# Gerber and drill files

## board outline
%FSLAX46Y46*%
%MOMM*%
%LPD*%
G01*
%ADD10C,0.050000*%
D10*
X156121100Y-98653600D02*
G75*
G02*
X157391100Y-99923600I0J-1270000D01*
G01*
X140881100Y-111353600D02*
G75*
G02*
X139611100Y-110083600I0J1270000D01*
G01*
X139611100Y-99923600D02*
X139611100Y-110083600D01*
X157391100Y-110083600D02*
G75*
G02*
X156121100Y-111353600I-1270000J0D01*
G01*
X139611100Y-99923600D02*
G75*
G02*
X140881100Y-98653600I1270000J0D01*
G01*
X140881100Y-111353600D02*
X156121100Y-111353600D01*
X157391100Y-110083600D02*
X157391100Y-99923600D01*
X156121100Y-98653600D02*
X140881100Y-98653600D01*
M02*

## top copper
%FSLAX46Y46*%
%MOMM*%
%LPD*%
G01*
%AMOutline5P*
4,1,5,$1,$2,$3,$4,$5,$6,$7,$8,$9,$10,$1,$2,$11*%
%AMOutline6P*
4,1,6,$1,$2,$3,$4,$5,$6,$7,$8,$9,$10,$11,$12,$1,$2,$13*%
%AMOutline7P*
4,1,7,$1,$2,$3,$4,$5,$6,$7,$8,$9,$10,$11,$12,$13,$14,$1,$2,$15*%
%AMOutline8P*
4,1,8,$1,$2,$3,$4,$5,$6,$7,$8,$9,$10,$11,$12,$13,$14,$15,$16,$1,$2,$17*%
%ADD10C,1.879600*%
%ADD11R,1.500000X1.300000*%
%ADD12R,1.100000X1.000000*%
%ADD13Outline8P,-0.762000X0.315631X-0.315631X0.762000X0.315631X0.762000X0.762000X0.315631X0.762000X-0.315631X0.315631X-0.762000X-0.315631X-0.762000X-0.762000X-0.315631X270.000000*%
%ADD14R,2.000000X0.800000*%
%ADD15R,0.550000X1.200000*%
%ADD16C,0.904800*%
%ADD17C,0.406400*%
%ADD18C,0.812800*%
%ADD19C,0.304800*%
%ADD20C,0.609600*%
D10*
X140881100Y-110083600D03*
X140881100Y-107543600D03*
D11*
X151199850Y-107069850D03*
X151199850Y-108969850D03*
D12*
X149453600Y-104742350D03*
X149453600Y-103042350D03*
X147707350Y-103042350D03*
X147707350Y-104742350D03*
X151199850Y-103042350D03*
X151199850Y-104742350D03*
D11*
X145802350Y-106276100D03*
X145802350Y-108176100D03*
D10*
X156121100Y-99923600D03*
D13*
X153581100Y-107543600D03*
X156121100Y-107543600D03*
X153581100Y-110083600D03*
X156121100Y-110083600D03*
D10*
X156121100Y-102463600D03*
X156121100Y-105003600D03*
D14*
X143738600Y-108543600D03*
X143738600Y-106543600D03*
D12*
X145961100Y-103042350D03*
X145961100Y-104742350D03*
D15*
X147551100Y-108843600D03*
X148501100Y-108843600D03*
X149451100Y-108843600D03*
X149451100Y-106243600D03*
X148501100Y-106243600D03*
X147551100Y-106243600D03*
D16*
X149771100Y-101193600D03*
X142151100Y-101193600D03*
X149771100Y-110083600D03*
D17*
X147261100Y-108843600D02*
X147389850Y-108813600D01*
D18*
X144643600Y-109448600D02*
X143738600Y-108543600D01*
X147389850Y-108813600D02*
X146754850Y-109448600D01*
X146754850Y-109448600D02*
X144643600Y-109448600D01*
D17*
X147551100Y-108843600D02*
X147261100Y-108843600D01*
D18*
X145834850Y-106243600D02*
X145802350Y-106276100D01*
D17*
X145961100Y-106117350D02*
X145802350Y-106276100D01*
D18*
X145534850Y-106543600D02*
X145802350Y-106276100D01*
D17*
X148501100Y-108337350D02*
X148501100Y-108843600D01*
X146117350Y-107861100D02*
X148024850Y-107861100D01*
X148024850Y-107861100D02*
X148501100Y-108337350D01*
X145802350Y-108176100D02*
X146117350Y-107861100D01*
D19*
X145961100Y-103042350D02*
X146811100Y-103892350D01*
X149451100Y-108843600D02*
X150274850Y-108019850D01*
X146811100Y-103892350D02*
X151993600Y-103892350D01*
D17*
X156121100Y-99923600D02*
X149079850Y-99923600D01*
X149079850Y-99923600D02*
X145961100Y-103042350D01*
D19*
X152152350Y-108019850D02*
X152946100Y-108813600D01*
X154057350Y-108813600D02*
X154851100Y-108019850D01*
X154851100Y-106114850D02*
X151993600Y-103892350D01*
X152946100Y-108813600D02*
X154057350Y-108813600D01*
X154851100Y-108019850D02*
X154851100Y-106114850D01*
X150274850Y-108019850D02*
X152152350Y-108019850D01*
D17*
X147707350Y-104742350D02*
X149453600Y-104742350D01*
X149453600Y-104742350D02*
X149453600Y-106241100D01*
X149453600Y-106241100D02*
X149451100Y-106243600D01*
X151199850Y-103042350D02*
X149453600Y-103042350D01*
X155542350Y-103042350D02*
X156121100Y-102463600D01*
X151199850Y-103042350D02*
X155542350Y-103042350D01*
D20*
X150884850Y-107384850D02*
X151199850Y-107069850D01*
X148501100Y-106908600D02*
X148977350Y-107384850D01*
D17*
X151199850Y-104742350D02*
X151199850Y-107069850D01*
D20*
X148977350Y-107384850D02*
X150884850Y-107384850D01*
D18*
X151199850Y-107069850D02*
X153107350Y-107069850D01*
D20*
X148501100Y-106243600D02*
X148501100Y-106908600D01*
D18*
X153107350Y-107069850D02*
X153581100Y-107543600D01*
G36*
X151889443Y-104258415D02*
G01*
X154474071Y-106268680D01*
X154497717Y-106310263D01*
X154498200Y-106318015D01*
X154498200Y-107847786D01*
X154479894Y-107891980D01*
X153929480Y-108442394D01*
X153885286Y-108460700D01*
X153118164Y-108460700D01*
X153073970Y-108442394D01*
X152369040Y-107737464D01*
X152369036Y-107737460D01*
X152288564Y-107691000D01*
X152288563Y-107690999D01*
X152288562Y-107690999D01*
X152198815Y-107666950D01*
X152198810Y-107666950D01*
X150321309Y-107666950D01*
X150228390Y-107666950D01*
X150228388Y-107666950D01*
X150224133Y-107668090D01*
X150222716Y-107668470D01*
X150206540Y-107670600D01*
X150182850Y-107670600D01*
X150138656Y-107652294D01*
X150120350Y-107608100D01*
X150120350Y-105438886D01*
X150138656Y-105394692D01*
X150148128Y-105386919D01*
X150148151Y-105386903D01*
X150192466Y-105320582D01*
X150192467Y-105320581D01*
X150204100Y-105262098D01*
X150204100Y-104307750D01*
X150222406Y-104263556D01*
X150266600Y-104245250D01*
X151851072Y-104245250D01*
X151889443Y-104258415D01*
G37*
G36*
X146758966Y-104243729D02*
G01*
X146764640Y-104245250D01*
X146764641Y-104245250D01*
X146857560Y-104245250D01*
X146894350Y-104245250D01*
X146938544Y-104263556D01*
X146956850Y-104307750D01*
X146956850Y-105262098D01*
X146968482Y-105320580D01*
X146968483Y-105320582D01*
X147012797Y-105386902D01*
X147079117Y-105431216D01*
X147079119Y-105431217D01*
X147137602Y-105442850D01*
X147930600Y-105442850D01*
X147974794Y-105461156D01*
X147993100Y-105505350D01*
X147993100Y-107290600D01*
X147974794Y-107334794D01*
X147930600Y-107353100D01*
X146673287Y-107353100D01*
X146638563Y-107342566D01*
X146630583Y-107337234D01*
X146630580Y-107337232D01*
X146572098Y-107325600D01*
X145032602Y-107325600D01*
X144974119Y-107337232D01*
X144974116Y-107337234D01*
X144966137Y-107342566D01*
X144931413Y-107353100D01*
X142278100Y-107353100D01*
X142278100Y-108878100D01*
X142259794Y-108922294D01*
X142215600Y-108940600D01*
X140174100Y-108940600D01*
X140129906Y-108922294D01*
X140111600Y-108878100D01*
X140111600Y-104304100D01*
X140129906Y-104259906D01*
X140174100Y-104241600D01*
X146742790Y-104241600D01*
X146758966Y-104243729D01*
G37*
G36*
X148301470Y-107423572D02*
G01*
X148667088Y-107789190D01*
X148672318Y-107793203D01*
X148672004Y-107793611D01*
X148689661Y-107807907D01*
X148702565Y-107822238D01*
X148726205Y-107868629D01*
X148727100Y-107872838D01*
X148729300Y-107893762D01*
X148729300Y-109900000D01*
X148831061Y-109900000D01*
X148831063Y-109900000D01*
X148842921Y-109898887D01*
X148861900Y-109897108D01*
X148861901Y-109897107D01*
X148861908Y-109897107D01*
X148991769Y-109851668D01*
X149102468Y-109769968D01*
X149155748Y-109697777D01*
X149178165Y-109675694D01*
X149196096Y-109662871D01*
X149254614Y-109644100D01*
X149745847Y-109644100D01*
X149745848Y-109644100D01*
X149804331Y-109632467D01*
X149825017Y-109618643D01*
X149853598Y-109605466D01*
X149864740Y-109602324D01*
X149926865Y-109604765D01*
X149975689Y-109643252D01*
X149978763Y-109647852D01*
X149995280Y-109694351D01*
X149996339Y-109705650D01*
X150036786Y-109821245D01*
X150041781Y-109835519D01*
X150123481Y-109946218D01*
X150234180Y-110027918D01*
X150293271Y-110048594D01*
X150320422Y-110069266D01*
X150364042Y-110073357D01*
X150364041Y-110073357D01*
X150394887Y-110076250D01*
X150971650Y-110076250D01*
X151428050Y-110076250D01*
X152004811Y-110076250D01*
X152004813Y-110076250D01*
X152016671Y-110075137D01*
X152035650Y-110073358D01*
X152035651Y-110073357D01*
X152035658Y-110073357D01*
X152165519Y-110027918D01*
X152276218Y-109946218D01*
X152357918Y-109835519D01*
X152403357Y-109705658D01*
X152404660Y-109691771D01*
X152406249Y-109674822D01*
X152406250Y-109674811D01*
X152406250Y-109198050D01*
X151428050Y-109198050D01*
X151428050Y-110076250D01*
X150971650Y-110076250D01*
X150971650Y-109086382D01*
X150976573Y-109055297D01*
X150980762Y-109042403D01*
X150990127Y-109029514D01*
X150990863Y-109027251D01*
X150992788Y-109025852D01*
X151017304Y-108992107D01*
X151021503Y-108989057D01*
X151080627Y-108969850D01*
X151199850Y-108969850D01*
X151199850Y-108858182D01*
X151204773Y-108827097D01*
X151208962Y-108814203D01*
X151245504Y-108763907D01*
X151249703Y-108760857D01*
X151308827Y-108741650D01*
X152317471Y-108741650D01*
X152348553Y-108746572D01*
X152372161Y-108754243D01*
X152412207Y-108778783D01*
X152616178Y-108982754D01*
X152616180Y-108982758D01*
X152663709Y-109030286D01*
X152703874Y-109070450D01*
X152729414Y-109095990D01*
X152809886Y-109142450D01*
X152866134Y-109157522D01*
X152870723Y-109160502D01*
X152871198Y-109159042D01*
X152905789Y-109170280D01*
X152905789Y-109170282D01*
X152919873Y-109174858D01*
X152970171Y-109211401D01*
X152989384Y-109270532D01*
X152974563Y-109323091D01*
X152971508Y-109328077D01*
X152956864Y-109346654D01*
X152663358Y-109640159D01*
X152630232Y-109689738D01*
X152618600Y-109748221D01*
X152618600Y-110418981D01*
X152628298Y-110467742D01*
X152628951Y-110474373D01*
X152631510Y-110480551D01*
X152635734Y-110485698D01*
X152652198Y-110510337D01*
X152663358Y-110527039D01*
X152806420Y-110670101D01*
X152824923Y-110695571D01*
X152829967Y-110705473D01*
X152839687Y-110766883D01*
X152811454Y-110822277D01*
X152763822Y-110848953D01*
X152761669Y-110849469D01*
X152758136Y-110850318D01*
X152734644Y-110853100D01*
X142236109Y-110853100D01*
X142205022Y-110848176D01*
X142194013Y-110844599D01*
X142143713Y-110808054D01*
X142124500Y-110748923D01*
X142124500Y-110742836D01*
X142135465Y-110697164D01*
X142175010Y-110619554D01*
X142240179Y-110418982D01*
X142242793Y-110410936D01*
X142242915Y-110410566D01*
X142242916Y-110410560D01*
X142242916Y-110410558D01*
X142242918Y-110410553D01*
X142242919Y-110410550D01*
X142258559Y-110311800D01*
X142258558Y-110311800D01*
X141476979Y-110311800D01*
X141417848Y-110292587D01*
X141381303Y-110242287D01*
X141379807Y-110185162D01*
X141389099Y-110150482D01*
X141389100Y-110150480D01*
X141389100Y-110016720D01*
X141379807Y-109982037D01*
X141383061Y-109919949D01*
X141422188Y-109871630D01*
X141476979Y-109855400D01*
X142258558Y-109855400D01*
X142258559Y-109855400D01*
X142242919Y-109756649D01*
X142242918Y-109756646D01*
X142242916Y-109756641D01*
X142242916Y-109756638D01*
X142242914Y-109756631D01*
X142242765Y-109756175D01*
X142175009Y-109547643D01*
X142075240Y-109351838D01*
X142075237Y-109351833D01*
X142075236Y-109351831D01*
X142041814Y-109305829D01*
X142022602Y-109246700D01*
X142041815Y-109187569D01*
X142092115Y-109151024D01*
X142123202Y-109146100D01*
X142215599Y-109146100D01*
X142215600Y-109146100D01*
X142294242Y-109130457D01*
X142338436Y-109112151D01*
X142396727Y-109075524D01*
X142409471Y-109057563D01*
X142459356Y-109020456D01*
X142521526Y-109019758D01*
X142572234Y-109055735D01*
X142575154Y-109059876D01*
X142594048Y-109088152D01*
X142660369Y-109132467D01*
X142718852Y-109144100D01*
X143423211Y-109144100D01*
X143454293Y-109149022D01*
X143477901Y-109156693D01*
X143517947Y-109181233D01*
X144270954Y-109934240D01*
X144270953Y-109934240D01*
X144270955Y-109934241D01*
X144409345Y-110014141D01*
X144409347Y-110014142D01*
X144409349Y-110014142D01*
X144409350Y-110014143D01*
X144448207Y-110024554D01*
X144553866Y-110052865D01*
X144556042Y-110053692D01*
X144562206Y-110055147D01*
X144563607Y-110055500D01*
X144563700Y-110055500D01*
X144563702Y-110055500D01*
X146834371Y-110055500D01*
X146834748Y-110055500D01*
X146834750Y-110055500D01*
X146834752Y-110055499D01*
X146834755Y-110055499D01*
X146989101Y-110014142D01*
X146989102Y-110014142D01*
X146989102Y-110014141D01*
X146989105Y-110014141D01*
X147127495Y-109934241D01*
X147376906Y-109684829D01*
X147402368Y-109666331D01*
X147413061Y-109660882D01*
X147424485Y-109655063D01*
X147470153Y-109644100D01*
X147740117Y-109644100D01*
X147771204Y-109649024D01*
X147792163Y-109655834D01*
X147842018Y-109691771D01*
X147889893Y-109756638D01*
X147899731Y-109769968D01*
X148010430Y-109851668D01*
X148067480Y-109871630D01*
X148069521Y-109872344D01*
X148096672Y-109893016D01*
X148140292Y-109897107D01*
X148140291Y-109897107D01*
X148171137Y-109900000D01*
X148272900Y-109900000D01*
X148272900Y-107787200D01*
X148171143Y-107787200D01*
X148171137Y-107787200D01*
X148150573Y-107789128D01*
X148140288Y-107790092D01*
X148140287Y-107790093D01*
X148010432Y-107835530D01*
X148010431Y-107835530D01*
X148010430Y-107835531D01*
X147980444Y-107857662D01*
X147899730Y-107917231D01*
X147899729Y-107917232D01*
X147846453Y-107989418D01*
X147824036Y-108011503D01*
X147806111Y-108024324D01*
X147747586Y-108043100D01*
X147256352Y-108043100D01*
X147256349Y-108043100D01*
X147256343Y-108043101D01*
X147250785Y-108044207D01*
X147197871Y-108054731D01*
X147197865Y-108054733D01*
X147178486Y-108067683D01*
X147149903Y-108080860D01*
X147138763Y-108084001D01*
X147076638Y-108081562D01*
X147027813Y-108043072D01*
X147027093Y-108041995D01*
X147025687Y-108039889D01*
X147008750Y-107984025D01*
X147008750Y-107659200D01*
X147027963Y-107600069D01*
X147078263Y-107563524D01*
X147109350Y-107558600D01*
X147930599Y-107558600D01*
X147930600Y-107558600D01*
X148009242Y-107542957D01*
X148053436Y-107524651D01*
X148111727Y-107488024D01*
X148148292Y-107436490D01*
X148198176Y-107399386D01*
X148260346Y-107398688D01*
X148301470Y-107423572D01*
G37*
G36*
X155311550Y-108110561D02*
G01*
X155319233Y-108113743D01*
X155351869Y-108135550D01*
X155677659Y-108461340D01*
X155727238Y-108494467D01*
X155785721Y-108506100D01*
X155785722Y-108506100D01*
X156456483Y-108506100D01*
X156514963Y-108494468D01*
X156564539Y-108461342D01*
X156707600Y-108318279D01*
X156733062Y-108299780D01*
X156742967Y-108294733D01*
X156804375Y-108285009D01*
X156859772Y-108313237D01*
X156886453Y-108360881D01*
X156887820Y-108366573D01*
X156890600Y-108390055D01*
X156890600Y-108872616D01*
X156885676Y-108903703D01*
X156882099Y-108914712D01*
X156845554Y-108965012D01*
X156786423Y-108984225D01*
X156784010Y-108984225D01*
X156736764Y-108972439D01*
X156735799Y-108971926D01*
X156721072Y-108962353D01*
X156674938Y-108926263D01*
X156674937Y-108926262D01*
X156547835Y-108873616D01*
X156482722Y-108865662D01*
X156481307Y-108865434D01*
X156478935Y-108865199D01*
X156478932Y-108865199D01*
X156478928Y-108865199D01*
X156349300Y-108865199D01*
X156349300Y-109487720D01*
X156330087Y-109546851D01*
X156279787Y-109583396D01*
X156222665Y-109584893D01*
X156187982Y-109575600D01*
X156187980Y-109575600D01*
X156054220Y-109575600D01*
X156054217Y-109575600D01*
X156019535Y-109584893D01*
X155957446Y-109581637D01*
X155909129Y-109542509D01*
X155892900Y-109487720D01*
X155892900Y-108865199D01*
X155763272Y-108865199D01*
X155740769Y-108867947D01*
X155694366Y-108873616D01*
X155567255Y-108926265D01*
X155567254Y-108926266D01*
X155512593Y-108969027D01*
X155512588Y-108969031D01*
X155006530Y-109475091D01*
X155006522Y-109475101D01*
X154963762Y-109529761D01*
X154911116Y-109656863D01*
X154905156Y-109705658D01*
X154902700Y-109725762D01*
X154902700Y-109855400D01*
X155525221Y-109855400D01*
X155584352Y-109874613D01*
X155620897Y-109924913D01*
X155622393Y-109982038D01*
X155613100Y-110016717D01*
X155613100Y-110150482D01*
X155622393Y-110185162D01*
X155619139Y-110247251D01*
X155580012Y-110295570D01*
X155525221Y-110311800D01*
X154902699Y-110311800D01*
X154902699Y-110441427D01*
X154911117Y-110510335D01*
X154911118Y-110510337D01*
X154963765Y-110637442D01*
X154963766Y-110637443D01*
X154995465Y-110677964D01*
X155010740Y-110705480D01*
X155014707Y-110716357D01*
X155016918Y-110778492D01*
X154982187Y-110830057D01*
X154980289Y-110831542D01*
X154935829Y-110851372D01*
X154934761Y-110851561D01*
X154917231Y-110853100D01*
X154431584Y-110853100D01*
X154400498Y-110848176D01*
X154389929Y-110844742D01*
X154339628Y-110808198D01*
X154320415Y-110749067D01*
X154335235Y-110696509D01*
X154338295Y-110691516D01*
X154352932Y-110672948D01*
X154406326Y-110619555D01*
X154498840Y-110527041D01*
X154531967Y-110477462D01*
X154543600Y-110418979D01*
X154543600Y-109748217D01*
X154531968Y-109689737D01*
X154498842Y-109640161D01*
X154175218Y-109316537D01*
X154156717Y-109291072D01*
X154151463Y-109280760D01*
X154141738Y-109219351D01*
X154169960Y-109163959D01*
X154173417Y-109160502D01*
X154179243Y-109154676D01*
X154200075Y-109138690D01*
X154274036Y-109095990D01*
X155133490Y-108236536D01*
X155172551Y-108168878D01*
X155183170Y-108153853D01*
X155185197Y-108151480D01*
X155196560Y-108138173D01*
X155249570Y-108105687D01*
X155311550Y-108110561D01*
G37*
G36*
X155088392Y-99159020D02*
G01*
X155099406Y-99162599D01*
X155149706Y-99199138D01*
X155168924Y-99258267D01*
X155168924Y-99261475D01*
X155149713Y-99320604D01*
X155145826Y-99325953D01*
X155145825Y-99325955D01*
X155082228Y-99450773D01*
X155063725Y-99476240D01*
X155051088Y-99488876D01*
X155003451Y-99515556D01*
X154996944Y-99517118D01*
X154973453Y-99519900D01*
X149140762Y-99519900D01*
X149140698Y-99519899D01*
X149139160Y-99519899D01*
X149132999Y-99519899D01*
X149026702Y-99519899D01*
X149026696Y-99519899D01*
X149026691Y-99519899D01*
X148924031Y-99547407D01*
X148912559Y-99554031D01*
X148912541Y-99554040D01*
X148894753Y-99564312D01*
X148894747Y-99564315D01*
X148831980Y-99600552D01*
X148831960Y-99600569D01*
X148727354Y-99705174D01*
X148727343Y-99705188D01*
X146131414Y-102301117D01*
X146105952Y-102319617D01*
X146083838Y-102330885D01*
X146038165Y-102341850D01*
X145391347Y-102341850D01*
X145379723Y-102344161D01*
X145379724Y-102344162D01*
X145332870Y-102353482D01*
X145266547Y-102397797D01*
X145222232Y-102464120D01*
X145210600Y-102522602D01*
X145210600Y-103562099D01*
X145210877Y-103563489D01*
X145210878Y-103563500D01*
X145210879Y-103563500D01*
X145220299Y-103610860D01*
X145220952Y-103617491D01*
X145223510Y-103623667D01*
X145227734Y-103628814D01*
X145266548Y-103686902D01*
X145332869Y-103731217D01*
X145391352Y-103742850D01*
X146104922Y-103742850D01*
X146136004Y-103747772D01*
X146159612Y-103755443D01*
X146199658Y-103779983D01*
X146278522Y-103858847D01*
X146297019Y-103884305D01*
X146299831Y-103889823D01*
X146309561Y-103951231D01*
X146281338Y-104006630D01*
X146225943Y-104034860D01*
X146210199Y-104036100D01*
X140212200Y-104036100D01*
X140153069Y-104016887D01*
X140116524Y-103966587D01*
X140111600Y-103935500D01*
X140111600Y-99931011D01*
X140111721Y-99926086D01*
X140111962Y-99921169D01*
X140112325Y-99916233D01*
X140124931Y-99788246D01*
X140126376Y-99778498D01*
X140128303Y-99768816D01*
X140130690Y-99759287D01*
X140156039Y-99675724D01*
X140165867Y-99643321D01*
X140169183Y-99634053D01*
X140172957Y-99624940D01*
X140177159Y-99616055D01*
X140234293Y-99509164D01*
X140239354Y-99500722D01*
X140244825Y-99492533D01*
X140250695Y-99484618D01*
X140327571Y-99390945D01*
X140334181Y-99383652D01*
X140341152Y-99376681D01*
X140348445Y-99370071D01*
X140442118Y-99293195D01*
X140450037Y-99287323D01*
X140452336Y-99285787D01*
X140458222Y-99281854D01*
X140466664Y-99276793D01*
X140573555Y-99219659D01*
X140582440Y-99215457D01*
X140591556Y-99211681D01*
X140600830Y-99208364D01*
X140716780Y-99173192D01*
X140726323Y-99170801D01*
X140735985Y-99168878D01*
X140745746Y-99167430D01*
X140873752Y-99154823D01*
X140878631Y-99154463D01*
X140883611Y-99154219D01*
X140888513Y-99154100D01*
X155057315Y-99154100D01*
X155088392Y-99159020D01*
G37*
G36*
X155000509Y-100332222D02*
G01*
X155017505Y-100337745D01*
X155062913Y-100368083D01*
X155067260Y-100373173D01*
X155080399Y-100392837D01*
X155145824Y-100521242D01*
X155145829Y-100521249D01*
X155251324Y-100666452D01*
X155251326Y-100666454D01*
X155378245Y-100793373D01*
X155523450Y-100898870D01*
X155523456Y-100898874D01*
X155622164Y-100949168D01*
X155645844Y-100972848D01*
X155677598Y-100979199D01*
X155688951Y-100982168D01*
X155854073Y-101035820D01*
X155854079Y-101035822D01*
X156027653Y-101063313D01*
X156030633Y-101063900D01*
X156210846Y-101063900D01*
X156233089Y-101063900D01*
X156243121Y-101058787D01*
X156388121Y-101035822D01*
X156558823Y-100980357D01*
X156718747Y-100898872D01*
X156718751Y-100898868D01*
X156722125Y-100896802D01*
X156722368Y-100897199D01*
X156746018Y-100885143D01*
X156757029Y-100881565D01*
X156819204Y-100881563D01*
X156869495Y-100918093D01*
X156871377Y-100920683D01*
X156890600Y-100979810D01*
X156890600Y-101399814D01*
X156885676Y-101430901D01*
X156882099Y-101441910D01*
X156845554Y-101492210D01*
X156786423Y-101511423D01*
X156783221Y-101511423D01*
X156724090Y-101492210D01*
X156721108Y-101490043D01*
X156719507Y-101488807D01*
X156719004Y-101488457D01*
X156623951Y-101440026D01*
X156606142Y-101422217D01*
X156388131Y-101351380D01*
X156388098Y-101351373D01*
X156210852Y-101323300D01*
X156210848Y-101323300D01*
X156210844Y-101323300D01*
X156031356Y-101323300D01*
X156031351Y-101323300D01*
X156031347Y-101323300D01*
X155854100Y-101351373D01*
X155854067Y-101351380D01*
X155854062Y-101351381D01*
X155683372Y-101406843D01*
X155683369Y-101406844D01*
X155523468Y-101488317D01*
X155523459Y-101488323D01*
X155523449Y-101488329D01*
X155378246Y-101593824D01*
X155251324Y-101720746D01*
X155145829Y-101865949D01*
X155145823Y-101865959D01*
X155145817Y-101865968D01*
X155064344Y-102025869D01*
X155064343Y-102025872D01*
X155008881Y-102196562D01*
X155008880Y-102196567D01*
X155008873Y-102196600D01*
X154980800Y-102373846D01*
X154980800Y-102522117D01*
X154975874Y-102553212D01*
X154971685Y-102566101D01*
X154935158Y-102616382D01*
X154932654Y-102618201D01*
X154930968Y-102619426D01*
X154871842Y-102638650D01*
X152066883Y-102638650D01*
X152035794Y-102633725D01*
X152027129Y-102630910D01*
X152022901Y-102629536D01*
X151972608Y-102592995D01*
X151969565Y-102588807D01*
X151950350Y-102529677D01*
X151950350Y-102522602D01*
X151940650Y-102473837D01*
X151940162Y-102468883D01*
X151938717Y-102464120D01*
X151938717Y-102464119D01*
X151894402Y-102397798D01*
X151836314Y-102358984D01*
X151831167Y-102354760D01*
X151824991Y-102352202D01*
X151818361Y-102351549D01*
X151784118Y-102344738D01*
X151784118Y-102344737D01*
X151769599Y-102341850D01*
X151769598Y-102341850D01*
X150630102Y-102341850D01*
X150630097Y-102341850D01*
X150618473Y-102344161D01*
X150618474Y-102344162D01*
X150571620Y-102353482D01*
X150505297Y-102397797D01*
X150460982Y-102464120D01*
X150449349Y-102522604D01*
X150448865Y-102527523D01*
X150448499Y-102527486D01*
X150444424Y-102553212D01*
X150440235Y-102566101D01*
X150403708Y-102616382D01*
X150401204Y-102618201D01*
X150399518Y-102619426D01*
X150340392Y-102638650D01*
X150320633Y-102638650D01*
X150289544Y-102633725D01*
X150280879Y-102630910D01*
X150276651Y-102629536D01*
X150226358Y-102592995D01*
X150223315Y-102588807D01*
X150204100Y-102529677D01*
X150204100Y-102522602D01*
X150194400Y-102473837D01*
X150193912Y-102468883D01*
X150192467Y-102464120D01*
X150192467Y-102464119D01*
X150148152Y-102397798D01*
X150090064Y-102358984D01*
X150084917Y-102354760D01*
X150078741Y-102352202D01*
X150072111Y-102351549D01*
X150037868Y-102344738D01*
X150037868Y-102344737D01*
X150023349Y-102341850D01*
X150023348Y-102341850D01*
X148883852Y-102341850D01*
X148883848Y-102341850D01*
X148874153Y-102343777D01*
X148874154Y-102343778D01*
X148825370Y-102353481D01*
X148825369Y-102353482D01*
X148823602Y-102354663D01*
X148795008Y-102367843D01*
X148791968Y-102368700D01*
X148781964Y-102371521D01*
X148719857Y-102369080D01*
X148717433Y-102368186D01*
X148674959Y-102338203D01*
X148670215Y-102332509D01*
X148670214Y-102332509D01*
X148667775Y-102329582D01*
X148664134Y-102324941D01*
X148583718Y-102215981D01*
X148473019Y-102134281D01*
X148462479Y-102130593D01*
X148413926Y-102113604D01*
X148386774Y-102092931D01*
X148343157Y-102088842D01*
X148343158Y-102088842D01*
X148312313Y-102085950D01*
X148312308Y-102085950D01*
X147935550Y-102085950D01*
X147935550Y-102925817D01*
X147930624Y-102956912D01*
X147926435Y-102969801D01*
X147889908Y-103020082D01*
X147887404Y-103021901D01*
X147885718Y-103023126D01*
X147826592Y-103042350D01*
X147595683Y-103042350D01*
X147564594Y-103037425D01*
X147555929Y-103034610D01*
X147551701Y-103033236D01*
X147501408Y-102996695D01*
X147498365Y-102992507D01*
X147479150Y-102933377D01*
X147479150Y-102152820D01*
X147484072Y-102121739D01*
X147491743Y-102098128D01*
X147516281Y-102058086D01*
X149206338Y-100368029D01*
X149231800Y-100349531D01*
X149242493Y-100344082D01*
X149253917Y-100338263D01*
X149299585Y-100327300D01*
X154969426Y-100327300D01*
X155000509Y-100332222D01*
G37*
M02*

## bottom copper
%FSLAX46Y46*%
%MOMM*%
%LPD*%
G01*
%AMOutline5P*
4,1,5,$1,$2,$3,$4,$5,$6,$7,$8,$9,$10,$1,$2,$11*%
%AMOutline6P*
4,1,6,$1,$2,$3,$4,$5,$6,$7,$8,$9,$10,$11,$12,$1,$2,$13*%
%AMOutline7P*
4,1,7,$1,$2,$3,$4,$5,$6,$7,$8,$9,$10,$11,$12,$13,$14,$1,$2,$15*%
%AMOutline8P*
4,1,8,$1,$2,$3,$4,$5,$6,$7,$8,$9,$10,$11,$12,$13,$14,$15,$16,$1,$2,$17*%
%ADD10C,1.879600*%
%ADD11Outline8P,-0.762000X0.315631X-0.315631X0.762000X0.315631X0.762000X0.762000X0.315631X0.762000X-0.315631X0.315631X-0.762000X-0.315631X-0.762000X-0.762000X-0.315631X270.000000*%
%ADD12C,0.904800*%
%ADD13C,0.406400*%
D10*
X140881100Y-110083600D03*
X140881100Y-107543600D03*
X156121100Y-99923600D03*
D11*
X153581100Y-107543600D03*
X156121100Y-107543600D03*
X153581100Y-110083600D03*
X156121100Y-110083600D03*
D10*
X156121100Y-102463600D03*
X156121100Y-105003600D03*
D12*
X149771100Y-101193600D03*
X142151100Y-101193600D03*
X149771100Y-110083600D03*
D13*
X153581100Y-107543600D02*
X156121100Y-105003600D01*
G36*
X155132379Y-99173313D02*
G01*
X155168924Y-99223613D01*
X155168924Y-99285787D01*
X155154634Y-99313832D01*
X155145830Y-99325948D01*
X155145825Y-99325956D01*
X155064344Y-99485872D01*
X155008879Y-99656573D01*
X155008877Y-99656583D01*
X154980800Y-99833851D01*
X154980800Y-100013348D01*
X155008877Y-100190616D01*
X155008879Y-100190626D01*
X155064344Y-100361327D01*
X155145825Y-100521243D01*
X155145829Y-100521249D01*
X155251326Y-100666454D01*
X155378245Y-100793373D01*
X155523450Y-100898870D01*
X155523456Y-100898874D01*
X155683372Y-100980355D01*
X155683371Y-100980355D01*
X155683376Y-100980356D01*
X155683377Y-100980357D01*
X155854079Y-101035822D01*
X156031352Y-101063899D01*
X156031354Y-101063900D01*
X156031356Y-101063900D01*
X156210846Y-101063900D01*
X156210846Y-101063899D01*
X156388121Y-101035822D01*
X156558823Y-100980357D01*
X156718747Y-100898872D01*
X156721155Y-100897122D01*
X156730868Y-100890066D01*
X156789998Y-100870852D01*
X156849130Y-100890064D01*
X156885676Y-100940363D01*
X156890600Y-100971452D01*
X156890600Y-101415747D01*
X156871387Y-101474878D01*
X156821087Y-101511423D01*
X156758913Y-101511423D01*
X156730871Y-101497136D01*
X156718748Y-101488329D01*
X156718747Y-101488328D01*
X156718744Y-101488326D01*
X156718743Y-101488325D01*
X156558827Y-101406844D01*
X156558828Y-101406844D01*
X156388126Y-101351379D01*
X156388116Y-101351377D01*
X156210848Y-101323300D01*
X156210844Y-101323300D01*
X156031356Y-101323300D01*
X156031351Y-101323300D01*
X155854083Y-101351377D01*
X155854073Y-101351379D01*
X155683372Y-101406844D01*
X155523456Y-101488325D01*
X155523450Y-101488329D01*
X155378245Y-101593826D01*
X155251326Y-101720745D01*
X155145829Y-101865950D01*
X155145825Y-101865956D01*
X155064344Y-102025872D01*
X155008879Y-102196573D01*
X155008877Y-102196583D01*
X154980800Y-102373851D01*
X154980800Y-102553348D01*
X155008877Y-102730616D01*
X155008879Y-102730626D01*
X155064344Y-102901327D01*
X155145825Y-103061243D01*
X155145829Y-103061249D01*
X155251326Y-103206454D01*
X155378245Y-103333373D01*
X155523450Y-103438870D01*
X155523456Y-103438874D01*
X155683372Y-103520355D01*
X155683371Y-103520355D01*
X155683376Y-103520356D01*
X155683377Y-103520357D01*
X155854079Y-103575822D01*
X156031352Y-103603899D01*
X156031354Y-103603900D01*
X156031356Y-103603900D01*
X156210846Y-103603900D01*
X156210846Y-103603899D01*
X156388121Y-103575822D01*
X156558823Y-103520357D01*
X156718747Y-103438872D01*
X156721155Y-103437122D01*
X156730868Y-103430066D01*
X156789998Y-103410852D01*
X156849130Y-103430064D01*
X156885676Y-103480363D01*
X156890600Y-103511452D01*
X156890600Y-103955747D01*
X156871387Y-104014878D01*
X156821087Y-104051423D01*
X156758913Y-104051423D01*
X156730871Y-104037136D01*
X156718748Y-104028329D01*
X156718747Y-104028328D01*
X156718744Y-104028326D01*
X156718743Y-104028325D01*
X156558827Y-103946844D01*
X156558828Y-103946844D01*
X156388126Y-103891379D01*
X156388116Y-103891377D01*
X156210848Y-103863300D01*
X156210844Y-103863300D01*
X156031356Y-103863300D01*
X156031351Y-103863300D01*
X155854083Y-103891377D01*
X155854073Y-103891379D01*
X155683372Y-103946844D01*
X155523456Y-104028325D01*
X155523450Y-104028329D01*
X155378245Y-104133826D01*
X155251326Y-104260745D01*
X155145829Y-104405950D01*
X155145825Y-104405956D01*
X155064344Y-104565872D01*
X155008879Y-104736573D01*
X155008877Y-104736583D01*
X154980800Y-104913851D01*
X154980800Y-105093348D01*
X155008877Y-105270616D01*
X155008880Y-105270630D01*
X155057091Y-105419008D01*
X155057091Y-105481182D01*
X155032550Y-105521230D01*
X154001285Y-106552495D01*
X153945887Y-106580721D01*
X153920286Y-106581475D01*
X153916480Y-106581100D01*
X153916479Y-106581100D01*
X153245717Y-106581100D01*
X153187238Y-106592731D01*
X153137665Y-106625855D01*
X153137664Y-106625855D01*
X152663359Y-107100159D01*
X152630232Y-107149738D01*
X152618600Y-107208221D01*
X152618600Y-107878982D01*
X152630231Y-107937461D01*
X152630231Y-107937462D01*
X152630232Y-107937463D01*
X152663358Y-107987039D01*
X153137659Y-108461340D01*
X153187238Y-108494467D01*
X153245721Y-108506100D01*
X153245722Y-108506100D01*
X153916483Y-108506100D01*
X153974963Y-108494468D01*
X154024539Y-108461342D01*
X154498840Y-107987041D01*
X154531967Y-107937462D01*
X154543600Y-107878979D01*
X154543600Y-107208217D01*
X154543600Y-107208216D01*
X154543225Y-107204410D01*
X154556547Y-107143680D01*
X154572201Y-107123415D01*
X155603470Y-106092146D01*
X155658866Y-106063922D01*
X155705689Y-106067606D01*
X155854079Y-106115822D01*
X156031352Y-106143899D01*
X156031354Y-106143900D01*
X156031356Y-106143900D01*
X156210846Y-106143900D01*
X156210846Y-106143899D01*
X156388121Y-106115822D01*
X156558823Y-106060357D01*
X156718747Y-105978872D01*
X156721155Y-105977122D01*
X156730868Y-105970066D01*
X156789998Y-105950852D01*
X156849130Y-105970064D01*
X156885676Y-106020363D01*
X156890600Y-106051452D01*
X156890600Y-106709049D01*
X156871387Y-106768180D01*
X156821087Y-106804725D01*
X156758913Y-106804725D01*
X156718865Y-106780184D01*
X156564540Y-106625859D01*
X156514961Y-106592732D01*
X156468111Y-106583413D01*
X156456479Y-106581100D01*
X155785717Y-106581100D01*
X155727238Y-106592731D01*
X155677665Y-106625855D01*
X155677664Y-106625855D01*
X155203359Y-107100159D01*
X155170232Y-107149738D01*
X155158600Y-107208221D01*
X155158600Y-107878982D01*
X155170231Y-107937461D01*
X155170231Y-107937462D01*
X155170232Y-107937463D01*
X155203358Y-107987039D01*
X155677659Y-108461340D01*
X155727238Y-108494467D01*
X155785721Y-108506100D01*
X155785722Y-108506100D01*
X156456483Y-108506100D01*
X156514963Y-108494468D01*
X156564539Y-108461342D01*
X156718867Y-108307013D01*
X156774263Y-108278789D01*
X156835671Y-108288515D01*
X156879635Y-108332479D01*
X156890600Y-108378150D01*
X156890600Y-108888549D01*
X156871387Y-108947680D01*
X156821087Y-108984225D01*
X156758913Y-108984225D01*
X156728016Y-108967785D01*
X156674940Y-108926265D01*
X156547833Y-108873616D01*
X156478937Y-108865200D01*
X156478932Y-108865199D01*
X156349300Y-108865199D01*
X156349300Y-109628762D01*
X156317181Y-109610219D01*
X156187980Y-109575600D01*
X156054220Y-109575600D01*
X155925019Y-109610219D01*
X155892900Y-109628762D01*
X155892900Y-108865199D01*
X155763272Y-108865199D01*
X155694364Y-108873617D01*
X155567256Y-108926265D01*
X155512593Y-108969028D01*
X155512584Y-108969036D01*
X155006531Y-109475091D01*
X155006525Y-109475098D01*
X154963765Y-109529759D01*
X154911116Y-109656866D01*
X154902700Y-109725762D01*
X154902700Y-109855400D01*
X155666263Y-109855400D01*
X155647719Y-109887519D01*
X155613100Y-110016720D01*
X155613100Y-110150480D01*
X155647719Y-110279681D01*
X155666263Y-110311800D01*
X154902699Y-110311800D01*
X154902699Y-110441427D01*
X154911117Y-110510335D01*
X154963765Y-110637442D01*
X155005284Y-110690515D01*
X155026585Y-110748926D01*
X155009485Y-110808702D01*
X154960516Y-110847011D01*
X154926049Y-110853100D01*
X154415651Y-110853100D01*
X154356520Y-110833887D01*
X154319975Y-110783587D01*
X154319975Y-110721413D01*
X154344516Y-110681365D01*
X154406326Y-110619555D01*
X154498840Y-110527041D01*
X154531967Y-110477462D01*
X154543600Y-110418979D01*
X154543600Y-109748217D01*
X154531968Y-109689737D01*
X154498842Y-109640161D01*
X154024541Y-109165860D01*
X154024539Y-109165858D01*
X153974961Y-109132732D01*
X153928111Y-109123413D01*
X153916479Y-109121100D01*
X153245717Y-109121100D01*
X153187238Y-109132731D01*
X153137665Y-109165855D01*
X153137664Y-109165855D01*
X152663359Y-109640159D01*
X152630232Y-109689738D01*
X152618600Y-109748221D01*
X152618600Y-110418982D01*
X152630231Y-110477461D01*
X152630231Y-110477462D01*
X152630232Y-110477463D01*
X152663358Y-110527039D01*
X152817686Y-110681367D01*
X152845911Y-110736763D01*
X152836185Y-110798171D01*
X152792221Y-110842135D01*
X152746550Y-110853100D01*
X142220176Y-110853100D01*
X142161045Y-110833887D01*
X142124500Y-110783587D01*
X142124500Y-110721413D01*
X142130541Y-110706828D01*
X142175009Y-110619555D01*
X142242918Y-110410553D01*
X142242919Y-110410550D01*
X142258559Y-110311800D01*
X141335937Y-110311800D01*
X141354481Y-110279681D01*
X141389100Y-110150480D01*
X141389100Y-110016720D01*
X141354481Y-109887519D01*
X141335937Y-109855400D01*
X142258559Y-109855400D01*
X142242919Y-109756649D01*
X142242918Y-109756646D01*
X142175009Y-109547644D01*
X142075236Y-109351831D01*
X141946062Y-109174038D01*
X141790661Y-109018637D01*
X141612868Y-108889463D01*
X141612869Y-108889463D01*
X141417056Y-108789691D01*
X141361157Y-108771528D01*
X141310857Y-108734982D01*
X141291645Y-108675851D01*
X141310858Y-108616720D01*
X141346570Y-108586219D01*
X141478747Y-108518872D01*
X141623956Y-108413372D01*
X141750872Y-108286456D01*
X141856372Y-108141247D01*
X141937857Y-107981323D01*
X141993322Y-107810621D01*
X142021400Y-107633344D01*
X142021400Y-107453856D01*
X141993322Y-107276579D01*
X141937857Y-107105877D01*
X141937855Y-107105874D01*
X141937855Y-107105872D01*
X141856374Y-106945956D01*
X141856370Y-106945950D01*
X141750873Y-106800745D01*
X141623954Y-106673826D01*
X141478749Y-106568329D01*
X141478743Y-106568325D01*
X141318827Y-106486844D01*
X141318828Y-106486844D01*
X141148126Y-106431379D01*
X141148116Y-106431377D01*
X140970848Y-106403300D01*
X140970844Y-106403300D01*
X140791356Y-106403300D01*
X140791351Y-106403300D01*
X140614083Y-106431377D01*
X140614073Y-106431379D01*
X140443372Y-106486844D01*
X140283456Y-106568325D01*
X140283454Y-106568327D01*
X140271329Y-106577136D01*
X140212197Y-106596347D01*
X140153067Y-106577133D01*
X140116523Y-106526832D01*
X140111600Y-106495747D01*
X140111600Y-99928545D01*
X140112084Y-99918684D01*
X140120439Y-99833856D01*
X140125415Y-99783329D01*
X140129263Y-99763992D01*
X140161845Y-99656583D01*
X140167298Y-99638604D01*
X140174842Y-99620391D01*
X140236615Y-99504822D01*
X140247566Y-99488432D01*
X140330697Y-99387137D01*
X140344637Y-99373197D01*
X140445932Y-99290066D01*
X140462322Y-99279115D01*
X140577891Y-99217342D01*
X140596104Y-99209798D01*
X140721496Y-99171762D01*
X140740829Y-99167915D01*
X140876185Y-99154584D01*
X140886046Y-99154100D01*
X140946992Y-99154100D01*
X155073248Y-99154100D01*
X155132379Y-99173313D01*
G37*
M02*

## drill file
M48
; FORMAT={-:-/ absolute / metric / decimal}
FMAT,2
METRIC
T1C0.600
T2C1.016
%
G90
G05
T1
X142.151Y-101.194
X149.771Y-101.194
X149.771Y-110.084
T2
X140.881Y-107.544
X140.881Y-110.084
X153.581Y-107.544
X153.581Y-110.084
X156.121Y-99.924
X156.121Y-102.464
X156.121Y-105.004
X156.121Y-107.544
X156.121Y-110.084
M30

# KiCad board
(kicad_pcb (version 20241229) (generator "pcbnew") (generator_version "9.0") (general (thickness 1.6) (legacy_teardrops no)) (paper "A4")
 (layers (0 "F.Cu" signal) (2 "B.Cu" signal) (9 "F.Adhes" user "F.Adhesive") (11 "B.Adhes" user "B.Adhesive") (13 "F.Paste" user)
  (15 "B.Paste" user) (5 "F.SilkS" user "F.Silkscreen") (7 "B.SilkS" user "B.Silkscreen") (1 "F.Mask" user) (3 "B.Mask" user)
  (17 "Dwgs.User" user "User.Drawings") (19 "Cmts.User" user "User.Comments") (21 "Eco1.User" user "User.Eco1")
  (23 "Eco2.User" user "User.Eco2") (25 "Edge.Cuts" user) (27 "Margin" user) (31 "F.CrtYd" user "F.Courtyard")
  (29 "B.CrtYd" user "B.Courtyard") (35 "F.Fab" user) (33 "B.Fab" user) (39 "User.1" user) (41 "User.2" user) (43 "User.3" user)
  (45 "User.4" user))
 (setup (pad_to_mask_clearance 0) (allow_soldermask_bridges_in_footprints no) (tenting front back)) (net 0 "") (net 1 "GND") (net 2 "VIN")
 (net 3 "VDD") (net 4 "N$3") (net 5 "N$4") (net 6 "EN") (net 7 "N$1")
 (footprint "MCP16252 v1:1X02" (layer "F.Cu") (at 140.8811 110.0836 90)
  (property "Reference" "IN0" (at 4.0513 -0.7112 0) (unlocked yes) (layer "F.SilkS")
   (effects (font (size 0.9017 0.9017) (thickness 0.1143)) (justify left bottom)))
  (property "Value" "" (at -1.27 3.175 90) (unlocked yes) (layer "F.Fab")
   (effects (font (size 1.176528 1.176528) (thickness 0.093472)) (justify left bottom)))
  (pad "1" thru_hole circle (at 0 0 180) (size 1.8796 1.8796) (drill 1.016) (layers "*.Cu" "*.Mask") (remove_unused_layers no) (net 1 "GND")
   (solder_mask_margin 0.0508) (thermal_bridge_angle 0))
  (pad "2" thru_hole circle (at 2.54 0 180) (size 1.8796 1.8796) (drill 1.016) (layers "*.Cu" "*.Mask") (remove_unused_layers no)
   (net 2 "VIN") (solder_mask_margin 0.0508) (thermal_bridge_angle 0)))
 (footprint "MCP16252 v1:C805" (layer "F.Cu") (at 151.19985 108.01985 -90)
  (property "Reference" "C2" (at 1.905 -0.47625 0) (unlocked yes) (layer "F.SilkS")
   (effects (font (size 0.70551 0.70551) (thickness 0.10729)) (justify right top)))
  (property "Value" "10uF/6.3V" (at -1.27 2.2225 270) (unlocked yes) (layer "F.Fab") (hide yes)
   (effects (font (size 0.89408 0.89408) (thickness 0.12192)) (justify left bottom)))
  (pad "1" smd rect (at -0.95 0 270) (size 1.3 1.5) (layers "F.Cu" "F.Mask" "F.Paste") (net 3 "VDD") (solder_mask_margin 0.0508)
   (solder_paste_margin 0) (thermal_bridge_angle 0))
  (pad "2" smd rect (at 0.95 0 270) (size 1.3 1.5) (layers "F.Cu" "F.Mask" "F.Paste") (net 1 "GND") (solder_mask_margin 0.0508)
   (solder_paste_margin 0) (thermal_bridge_angle 0)))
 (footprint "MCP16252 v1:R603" (layer "F.Cu") (at 149.4536 103.89235 90)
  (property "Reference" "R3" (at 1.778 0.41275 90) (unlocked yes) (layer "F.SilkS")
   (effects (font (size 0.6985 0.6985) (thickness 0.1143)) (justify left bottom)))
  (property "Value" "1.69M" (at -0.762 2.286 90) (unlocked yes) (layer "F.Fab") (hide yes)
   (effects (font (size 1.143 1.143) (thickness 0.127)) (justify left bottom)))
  (pad "1" smd rect (at -0.85 0 90) (size 1 1.1) (layers "F.Cu" "F.Mask" "F.Paste") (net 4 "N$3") (solder_mask_margin 0.0508)
   (solder_paste_margin 0) (thermal_bridge_angle 0))
  (pad "2" smd rect (at 0.85 0 90) (size 1 1.1) (layers "F.Cu" "F.Mask" "F.Paste") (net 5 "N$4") (solder_mask_margin 0.0508)
   (solder_paste_margin 0) (thermal_bridge_angle 0)))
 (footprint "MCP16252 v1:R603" (layer "F.Cu") (at 147.70735 103.89235 -90)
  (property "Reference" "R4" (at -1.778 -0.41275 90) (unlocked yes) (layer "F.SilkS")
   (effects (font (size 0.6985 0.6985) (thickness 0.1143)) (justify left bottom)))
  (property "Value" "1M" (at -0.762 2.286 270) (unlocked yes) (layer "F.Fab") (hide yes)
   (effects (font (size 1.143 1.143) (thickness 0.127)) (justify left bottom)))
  (pad "1" smd rect (at -0.85 0 270) (size 1 1.1) (layers "F.Cu" "F.Mask" "F.Paste") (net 1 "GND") (solder_mask_margin 0.0508)
   (solder_paste_margin 0) (thermal_bridge_angle 0))
  (pad "2" smd rect (at 0.85 0 270) (size 1 1.1) (layers "F.Cu" "F.Mask" "F.Paste") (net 4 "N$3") (solder_mask_margin 0.0508)
   (solder_paste_margin 0) (thermal_bridge_angle 0)))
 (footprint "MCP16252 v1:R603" (layer "F.Cu") (at 151.19985 103.89235 -90)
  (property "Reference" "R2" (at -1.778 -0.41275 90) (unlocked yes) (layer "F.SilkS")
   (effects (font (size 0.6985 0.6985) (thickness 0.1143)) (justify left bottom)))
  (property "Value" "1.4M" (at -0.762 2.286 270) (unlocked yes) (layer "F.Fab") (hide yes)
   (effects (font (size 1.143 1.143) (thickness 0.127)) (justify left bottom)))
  (pad "1" smd rect (at -0.85 0 270) (size 1 1.1) (layers "F.Cu" "F.Mask" "F.Paste") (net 5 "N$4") (solder_mask_margin 0.0508)
   (solder_paste_margin 0) (thermal_bridge_angle 0))
  (pad "2" smd rect (at 0.85 0 270) (size 1 1.1) (layers "F.Cu" "F.Mask" "F.Paste") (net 3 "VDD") (solder_mask_margin 0.0508)
   (solder_paste_margin 0) (thermal_bridge_angle 0)))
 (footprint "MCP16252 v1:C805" (layer "F.Cu") (at 145.80235 107.2261 -90)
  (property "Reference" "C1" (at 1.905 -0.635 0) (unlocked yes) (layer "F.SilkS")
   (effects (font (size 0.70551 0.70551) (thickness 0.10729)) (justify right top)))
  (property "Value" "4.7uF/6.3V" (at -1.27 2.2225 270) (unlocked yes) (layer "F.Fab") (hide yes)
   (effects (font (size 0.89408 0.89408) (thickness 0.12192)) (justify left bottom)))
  (pad "1" smd rect (at -0.95 0 270) (size 1.3 1.5) (layers "F.Cu" "F.Mask" "F.Paste") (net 2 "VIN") (solder_mask_margin 0.0508)
   (solder_paste_margin 0) (thermal_bridge_angle 0))
  (pad "2" smd rect (at 0.95 0 270) (size 1.3 1.5) (layers "F.Cu" "F.Mask" "F.Paste") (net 1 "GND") (solder_mask_margin 0.0508)
   (solder_paste_margin 0) (thermal_bridge_angle 0)))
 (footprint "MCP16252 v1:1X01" (layer "F.Cu") (at 156.1211 99.9236)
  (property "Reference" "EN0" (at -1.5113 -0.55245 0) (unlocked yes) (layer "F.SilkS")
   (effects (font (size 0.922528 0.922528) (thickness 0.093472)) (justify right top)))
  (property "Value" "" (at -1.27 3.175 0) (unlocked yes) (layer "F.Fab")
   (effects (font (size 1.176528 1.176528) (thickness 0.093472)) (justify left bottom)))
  (pad "1" thru_hole circle (at 0 0 90) (size 1.8796 1.8796) (drill 1.016) (layers "*.Cu" "*.Mask") (remove_unused_layers no) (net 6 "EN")
   (solder_mask_margin 0.0508) (thermal_bridge_angle 0)))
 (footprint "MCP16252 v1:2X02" (layer "F.Cu") (at 154.8511 108.8136 -90)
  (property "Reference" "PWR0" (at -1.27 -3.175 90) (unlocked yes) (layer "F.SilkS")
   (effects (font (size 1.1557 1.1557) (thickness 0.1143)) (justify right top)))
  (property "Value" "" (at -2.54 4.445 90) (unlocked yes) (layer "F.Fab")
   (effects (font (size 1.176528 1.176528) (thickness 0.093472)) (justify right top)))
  (pad "1" thru_hole roundrect (at -1.27 1.27 270) (size 1.524 1.524) (drill 1.016) (layers "*.Cu" "*.Mask") (remove_unused_layers no)
   (roundrect_rratio 0.25) (chamfer_ratio 0.2928932188) (chamfer top_left top_right bottom_left bottom_right) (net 3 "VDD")
   (solder_mask_margin 0.0508) (thermal_bridge_angle 0))
  (pad "2" thru_hole roundrect (at -1.27 -1.27 270) (size 1.524 1.524) (drill 1.016) (layers "*.Cu" "*.Mask") (remove_unused_layers no)
   (roundrect_rratio 0.25) (chamfer_ratio 0.2928932188) (chamfer top_left top_right bottom_left bottom_right) (solder_mask_margin 0.0508)
   (thermal_bridge_angle 0))
  (pad "3" thru_hole roundrect (at 1.27 1.27 270) (size 1.524 1.524) (drill 1.016) (layers "*.Cu" "*.Mask") (remove_unused_layers no)
   (roundrect_rratio 0.25) (chamfer_ratio 0.2928932188) (chamfer top_left top_right bottom_left bottom_right) (solder_mask_margin 0.0508)
   (thermal_bridge_angle 0))
  (pad "4" thru_hole roundrect (at 1.27 -1.27 270) (size 1.524 1.524) (drill 1.016) (layers "*.Cu" "*.Mask") (remove_unused_layers no)
   (roundrect_rratio 0.25) (chamfer_ratio 0.2928932188) (chamfer top_left top_right bottom_left bottom_right) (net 1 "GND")
   (solder_mask_margin 0.0508) (thermal_bridge_angle 0)))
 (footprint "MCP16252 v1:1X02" (layer "F.Cu") (at 156.1211 102.4636 -90)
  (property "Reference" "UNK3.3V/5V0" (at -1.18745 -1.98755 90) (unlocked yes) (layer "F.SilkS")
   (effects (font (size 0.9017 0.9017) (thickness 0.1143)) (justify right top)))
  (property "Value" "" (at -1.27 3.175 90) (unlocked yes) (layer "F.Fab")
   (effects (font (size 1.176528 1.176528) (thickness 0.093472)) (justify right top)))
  (pad "1" thru_hole circle (at 0 0) (size 1.8796 1.8796) (drill 1.016) (layers "*.Cu" "*.Mask") (remove_unused_layers no) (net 5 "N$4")
   (solder_mask_margin 0.0508) (thermal_bridge_angle 0))
  (pad "2" thru_hole circle (at 2.54 0) (size 1.8796 1.8796) (drill 1.016) (layers "*.Cu" "*.Mask") (remove_unused_layers no) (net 3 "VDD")
   (solder_mask_margin 0.0508) (thermal_bridge_angle 0)))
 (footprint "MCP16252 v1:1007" (layer "F.Cu") (at 143.7386 107.5436 180)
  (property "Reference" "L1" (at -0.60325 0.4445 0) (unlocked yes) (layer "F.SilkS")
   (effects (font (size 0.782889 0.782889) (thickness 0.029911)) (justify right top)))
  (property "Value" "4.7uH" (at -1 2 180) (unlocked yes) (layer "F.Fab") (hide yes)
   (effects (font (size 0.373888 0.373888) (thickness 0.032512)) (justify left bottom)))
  (pad "1" smd rect (at 0 -1 180) (size 2 0.8) (layers "F.Cu" "F.Mask" "F.Paste") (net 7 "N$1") (solder_mask_margin 0.0508)
   (solder_paste_margin 0) (thermal_bridge_angle 0))
  (pad "2" smd rect (at 0 1 180) (size 2 0.8) (layers "F.Cu" "F.Mask" "F.Paste") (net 2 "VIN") (solder_mask_margin 0.0508)
   (solder_paste_margin 0) (thermal_bridge_angle 0)))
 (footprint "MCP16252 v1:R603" (layer "F.Cu") (at 145.9611 103.89235 -90)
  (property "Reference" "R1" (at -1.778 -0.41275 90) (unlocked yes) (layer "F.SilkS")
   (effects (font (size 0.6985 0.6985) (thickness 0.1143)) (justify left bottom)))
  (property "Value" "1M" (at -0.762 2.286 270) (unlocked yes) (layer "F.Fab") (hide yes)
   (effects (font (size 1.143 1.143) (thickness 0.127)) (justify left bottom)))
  (pad "1" smd rect (at -0.85 0 270) (size 1 1.1) (layers "F.Cu" "F.Mask" "F.Paste") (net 6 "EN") (solder_mask_margin 0.0508)
   (solder_paste_margin 0) (thermal_bridge_angle 0))
  (pad "2" smd rect (at 0.85 0 270) (size 1 1.1) (layers "F.Cu" "F.Mask" "F.Paste") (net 2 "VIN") (solder_mask_margin 0.0508)
   (solder_paste_margin 0) (thermal_bridge_angle 0)))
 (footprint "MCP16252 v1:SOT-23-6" (layer "F.Cu") (at 148.5011 107.5436)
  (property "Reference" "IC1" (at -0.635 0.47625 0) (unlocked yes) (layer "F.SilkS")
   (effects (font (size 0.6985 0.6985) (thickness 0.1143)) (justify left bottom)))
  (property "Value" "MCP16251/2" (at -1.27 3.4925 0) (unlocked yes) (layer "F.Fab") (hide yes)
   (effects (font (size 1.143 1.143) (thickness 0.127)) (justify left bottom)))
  (pad "1" smd rect (at -0.95 1.3) (size 0.55 1.2) (layers "F.Cu" "F.Mask" "F.Paste") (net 7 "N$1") (solder_mask_margin 0.0508)
   (solder_paste_margin 0) (thermal_bridge_angle 0))
  (pad "2" smd rect (at 0 1.3) (size 0.55 1.2) (layers "F.Cu" "F.Mask" "F.Paste") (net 1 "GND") (solder_mask_margin 0.0508)
   (solder_paste_margin 0) (thermal_bridge_angle 0))
  (pad "3" smd rect (at 0.95 1.3) (size 0.55 1.2) (layers "F.Cu" "F.Mask" "F.Paste") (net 6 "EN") (solder_mask_margin 0.0508)
   (solder_paste_margin 0) (thermal_bridge_angle 0))
  (pad "4" smd rect (at 0.95 -1.3) (size 0.55 1.2) (layers "F.Cu" "F.Mask" "F.Paste") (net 4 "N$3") (solder_mask_margin 0.0508)
   (solder_paste_margin 0) (thermal_bridge_angle 0))
  (pad "5" smd rect (at 0 -1.3) (size 0.55 1.2) (layers "F.Cu" "F.Mask" "F.Paste") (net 3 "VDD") (solder_mask_margin 0.0508)
   (solder_paste_margin 0) (thermal_bridge_angle 0))
  (pad "6" smd rect (at -0.95 -1.3) (size 0.55 1.2) (layers "F.Cu" "F.Mask" "F.Paste") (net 2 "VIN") (solder_mask_margin 0.0508)
   (solder_paste_margin 0) (thermal_bridge_angle 0)))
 (gr_arc (start 156.1211 98.6536) (mid 157.019126 99.025574) (end 157.3911 99.9236) (stroke (width 0.05) (type solid)) (layer "Edge.Cuts"))
 (gr_arc (start 140.8811 111.3536) (mid 139.983074 110.981626) (end 139.6111 110.0836) (stroke (width 0.05) (type solid))
  (layer "Edge.Cuts"))
 (gr_line (start 139.6111 99.9236) (end 139.6111 110.0836) (stroke (width 0.05) (type solid)) (layer "Edge.Cuts"))
 (gr_arc (start 157.3911 110.0836) (mid 157.019126 110.981626) (end 156.1211 111.3536) (stroke (width 0.05) (type solid))
  (layer "Edge.Cuts"))
 (gr_arc (start 139.6111 99.9236) (mid 139.983074 99.025574) (end 140.8811 98.6536) (stroke (width 0.05) (type solid)) (layer "Edge.Cuts"))
 (gr_line (start 140.8811 111.3536) (end 156.1211 111.3536) (stroke (width 0.05) (type solid)) (layer "Edge.Cuts"))
 (gr_line (start 157.3911 110.0836) (end 157.3911 99.9236) (stroke (width 0.05) (type solid)) (layer "Edge.Cuts"))
 (gr_line (start 156.1211 98.6536) (end 140.8811 98.6536) (stroke (width 0.05) (type solid)) (layer "Edge.Cuts"))
 (segment (start 147.2611 108.8436) (end 147.38985 108.8136) (width 0.4064) (layer "F.Cu") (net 7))
 (segment (start 144.6436 109.4486) (end 143.7386 108.5436) (width 0.8128) (layer "F.Cu") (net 7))
 (segment (start 147.38985 108.8136) (end 146.75485 109.4486) (width 0.8128) (layer "F.Cu") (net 7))
 (segment (start 146.75485 109.4486) (end 144.6436 109.4486) (width 0.8128) (layer "F.Cu") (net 7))
 (segment (start 147.5511 108.8436) (end 147.2611 108.8436) (width 0.4064) (layer "F.Cu") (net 7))
 (segment (start 145.83485 106.2436) (end 145.80235 106.2761) (width 0.8128) (layer "F.Cu") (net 2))
 (segment (start 145.9611 106.11735) (end 145.80235 106.2761) (width 0.4064) (layer "F.Cu") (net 2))
 (segment (start 145.53485 106.5436) (end 145.80235 106.2761) (width 0.8128) (layer "F.Cu") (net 2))
 (segment (start 148.5011 108.33735) (end 148.5011 108.8436) (width 0.4064) (layer "F.Cu") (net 1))
 (segment (start 146.11735 107.8611) (end 148.02485 107.8611) (width 0.4064) (layer "F.Cu") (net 1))
 (segment (start 148.02485 107.8611) (end 148.5011 108.33735) (width 0.4064) (layer "F.Cu") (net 1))
 (segment (start 145.80235 108.1761) (end 146.11735 107.8611) (width 0.4064) (layer "F.Cu") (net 1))
 (via (at 149.7711 101.1936) (size 0.9048) (drill 0.6) (layers "F.Cu" "B.Cu") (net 1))
 (via (at 142.1511 101.1936) (size 0.9048) (drill 0.6) (layers "F.Cu" "B.Cu") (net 1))
 (via (at 149.7711 110.0836) (size 0.9048) (drill 0.6) (layers "F.Cu" "B.Cu") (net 1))
 (segment (start 145.9611 103.04235) (end 146.8111 103.89235) (width 0.3048) (layer "F.Cu") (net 6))
 (segment (start 149.4511 108.8436) (end 150.27485 108.01985) (width 0.3048) (layer "F.Cu") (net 6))
 (segment (start 146.8111 103.89235) (end 151.9936 103.89235) (width 0.3048) (layer "F.Cu") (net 6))
 (segment (start 156.1211 99.9236) (end 149.07985 99.9236) (width 0.4064) (layer "F.Cu") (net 6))
 (segment (start 149.07985 99.9236) (end 145.9611 103.04235) (width 0.4064) (layer "F.Cu") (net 6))
 (segment (start 152.15235 108.01985) (end 152.9461 108.8136) (width 0.3048) (layer "F.Cu") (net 6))
 (segment (start 154.05735 108.8136) (end 154.8511 108.01985) (width 0.3048) (layer "F.Cu") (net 6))
 (segment (start 154.8511 106.11485) (end 151.9936 103.89235) (width 0.3048) (layer "F.Cu") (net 6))
 (segment (start 152.9461 108.8136) (end 154.05735 108.8136) (width 0.3048) (layer "F.Cu") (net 6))
 (segment (start 154.8511 108.01985) (end 154.8511 106.11485) (width 0.3048) (layer "F.Cu") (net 6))
 (segment (start 150.27485 108.01985) (end 152.15235 108.01985) (width 0.3048) (layer "F.Cu") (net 6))
 (segment (start 147.70735 104.74235) (end 149.4536 104.74235) (width 0.4064) (layer "F.Cu") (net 4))
 (segment (start 149.4536 104.74235) (end 149.4536 106.2411) (width 0.4064) (layer "F.Cu") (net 4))
 (segment (start 149.4536 106.2411) (end 149.4511 106.2436) (width 0.4064) (layer "F.Cu") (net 4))
 (segment (start 151.19985 103.04235) (end 149.4536 103.04235) (width 0.4064) (layer "F.Cu") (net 5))
 (segment (start 155.54235 103.04235) (end 156.1211 102.4636) (width 0.4064) (layer "F.Cu") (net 5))
 (segment (start 151.19985 103.04235) (end 155.54235 103.04235) (width 0.4064) (layer "F.Cu") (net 5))
 (segment (start 150.88485 107.38485) (end 151.19985 107.06985) (width 0.6096) (layer "F.Cu") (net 3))
 (segment (start 148.5011 106.9086) (end 148.97735 107.38485) (width 0.6096) (layer "F.Cu") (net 3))
 (segment (start 151.19985 104.74235) (end 151.19985 107.06985) (width 0.4064) (layer "F.Cu") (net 3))
 (segment (start 148.97735 107.38485) (end 150.88485 107.38485) (width 0.6096) (layer "F.Cu") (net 3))
 (segment (start 151.19985 107.06985) (end 153.10735 107.06985) (width 0.8128) (layer "F.Cu") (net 3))
 (segment (start 148.5011 106.2436) (end 148.5011 106.9086) (width 0.6096) (layer "F.Cu") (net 3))
 (segment (start 153.10735 107.06985) (end 153.5811 107.5436) (width 0.8128) (layer "F.Cu") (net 3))
 (segment (start 153.5811 107.5436) (end 156.1211 105.0036) (width 0.4064) (layer "B.Cu") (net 3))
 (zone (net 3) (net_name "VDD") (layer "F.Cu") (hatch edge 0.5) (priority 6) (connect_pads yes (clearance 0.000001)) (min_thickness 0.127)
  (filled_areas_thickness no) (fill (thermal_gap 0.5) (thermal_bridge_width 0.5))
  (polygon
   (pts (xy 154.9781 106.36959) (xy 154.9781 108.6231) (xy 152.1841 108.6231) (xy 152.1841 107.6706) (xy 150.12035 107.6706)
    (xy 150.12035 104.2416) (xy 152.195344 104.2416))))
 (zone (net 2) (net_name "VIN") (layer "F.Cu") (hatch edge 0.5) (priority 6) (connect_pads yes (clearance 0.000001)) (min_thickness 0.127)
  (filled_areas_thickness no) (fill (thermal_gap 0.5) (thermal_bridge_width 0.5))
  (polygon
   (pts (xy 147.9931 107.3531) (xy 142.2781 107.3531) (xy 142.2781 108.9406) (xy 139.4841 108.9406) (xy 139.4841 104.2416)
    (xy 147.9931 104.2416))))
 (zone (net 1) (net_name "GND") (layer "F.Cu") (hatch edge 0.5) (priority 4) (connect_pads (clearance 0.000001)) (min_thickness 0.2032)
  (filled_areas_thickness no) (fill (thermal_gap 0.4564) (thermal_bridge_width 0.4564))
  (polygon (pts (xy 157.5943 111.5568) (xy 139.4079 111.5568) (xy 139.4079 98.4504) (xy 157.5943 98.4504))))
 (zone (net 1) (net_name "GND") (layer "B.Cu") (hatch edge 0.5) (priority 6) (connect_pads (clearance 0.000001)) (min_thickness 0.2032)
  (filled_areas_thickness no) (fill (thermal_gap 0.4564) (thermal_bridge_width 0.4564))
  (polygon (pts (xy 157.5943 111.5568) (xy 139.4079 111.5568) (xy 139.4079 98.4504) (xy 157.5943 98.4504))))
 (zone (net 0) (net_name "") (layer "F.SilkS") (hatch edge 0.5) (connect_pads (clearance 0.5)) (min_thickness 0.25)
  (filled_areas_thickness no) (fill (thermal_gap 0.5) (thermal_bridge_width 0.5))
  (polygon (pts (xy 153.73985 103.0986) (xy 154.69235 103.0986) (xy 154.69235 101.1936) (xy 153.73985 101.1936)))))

